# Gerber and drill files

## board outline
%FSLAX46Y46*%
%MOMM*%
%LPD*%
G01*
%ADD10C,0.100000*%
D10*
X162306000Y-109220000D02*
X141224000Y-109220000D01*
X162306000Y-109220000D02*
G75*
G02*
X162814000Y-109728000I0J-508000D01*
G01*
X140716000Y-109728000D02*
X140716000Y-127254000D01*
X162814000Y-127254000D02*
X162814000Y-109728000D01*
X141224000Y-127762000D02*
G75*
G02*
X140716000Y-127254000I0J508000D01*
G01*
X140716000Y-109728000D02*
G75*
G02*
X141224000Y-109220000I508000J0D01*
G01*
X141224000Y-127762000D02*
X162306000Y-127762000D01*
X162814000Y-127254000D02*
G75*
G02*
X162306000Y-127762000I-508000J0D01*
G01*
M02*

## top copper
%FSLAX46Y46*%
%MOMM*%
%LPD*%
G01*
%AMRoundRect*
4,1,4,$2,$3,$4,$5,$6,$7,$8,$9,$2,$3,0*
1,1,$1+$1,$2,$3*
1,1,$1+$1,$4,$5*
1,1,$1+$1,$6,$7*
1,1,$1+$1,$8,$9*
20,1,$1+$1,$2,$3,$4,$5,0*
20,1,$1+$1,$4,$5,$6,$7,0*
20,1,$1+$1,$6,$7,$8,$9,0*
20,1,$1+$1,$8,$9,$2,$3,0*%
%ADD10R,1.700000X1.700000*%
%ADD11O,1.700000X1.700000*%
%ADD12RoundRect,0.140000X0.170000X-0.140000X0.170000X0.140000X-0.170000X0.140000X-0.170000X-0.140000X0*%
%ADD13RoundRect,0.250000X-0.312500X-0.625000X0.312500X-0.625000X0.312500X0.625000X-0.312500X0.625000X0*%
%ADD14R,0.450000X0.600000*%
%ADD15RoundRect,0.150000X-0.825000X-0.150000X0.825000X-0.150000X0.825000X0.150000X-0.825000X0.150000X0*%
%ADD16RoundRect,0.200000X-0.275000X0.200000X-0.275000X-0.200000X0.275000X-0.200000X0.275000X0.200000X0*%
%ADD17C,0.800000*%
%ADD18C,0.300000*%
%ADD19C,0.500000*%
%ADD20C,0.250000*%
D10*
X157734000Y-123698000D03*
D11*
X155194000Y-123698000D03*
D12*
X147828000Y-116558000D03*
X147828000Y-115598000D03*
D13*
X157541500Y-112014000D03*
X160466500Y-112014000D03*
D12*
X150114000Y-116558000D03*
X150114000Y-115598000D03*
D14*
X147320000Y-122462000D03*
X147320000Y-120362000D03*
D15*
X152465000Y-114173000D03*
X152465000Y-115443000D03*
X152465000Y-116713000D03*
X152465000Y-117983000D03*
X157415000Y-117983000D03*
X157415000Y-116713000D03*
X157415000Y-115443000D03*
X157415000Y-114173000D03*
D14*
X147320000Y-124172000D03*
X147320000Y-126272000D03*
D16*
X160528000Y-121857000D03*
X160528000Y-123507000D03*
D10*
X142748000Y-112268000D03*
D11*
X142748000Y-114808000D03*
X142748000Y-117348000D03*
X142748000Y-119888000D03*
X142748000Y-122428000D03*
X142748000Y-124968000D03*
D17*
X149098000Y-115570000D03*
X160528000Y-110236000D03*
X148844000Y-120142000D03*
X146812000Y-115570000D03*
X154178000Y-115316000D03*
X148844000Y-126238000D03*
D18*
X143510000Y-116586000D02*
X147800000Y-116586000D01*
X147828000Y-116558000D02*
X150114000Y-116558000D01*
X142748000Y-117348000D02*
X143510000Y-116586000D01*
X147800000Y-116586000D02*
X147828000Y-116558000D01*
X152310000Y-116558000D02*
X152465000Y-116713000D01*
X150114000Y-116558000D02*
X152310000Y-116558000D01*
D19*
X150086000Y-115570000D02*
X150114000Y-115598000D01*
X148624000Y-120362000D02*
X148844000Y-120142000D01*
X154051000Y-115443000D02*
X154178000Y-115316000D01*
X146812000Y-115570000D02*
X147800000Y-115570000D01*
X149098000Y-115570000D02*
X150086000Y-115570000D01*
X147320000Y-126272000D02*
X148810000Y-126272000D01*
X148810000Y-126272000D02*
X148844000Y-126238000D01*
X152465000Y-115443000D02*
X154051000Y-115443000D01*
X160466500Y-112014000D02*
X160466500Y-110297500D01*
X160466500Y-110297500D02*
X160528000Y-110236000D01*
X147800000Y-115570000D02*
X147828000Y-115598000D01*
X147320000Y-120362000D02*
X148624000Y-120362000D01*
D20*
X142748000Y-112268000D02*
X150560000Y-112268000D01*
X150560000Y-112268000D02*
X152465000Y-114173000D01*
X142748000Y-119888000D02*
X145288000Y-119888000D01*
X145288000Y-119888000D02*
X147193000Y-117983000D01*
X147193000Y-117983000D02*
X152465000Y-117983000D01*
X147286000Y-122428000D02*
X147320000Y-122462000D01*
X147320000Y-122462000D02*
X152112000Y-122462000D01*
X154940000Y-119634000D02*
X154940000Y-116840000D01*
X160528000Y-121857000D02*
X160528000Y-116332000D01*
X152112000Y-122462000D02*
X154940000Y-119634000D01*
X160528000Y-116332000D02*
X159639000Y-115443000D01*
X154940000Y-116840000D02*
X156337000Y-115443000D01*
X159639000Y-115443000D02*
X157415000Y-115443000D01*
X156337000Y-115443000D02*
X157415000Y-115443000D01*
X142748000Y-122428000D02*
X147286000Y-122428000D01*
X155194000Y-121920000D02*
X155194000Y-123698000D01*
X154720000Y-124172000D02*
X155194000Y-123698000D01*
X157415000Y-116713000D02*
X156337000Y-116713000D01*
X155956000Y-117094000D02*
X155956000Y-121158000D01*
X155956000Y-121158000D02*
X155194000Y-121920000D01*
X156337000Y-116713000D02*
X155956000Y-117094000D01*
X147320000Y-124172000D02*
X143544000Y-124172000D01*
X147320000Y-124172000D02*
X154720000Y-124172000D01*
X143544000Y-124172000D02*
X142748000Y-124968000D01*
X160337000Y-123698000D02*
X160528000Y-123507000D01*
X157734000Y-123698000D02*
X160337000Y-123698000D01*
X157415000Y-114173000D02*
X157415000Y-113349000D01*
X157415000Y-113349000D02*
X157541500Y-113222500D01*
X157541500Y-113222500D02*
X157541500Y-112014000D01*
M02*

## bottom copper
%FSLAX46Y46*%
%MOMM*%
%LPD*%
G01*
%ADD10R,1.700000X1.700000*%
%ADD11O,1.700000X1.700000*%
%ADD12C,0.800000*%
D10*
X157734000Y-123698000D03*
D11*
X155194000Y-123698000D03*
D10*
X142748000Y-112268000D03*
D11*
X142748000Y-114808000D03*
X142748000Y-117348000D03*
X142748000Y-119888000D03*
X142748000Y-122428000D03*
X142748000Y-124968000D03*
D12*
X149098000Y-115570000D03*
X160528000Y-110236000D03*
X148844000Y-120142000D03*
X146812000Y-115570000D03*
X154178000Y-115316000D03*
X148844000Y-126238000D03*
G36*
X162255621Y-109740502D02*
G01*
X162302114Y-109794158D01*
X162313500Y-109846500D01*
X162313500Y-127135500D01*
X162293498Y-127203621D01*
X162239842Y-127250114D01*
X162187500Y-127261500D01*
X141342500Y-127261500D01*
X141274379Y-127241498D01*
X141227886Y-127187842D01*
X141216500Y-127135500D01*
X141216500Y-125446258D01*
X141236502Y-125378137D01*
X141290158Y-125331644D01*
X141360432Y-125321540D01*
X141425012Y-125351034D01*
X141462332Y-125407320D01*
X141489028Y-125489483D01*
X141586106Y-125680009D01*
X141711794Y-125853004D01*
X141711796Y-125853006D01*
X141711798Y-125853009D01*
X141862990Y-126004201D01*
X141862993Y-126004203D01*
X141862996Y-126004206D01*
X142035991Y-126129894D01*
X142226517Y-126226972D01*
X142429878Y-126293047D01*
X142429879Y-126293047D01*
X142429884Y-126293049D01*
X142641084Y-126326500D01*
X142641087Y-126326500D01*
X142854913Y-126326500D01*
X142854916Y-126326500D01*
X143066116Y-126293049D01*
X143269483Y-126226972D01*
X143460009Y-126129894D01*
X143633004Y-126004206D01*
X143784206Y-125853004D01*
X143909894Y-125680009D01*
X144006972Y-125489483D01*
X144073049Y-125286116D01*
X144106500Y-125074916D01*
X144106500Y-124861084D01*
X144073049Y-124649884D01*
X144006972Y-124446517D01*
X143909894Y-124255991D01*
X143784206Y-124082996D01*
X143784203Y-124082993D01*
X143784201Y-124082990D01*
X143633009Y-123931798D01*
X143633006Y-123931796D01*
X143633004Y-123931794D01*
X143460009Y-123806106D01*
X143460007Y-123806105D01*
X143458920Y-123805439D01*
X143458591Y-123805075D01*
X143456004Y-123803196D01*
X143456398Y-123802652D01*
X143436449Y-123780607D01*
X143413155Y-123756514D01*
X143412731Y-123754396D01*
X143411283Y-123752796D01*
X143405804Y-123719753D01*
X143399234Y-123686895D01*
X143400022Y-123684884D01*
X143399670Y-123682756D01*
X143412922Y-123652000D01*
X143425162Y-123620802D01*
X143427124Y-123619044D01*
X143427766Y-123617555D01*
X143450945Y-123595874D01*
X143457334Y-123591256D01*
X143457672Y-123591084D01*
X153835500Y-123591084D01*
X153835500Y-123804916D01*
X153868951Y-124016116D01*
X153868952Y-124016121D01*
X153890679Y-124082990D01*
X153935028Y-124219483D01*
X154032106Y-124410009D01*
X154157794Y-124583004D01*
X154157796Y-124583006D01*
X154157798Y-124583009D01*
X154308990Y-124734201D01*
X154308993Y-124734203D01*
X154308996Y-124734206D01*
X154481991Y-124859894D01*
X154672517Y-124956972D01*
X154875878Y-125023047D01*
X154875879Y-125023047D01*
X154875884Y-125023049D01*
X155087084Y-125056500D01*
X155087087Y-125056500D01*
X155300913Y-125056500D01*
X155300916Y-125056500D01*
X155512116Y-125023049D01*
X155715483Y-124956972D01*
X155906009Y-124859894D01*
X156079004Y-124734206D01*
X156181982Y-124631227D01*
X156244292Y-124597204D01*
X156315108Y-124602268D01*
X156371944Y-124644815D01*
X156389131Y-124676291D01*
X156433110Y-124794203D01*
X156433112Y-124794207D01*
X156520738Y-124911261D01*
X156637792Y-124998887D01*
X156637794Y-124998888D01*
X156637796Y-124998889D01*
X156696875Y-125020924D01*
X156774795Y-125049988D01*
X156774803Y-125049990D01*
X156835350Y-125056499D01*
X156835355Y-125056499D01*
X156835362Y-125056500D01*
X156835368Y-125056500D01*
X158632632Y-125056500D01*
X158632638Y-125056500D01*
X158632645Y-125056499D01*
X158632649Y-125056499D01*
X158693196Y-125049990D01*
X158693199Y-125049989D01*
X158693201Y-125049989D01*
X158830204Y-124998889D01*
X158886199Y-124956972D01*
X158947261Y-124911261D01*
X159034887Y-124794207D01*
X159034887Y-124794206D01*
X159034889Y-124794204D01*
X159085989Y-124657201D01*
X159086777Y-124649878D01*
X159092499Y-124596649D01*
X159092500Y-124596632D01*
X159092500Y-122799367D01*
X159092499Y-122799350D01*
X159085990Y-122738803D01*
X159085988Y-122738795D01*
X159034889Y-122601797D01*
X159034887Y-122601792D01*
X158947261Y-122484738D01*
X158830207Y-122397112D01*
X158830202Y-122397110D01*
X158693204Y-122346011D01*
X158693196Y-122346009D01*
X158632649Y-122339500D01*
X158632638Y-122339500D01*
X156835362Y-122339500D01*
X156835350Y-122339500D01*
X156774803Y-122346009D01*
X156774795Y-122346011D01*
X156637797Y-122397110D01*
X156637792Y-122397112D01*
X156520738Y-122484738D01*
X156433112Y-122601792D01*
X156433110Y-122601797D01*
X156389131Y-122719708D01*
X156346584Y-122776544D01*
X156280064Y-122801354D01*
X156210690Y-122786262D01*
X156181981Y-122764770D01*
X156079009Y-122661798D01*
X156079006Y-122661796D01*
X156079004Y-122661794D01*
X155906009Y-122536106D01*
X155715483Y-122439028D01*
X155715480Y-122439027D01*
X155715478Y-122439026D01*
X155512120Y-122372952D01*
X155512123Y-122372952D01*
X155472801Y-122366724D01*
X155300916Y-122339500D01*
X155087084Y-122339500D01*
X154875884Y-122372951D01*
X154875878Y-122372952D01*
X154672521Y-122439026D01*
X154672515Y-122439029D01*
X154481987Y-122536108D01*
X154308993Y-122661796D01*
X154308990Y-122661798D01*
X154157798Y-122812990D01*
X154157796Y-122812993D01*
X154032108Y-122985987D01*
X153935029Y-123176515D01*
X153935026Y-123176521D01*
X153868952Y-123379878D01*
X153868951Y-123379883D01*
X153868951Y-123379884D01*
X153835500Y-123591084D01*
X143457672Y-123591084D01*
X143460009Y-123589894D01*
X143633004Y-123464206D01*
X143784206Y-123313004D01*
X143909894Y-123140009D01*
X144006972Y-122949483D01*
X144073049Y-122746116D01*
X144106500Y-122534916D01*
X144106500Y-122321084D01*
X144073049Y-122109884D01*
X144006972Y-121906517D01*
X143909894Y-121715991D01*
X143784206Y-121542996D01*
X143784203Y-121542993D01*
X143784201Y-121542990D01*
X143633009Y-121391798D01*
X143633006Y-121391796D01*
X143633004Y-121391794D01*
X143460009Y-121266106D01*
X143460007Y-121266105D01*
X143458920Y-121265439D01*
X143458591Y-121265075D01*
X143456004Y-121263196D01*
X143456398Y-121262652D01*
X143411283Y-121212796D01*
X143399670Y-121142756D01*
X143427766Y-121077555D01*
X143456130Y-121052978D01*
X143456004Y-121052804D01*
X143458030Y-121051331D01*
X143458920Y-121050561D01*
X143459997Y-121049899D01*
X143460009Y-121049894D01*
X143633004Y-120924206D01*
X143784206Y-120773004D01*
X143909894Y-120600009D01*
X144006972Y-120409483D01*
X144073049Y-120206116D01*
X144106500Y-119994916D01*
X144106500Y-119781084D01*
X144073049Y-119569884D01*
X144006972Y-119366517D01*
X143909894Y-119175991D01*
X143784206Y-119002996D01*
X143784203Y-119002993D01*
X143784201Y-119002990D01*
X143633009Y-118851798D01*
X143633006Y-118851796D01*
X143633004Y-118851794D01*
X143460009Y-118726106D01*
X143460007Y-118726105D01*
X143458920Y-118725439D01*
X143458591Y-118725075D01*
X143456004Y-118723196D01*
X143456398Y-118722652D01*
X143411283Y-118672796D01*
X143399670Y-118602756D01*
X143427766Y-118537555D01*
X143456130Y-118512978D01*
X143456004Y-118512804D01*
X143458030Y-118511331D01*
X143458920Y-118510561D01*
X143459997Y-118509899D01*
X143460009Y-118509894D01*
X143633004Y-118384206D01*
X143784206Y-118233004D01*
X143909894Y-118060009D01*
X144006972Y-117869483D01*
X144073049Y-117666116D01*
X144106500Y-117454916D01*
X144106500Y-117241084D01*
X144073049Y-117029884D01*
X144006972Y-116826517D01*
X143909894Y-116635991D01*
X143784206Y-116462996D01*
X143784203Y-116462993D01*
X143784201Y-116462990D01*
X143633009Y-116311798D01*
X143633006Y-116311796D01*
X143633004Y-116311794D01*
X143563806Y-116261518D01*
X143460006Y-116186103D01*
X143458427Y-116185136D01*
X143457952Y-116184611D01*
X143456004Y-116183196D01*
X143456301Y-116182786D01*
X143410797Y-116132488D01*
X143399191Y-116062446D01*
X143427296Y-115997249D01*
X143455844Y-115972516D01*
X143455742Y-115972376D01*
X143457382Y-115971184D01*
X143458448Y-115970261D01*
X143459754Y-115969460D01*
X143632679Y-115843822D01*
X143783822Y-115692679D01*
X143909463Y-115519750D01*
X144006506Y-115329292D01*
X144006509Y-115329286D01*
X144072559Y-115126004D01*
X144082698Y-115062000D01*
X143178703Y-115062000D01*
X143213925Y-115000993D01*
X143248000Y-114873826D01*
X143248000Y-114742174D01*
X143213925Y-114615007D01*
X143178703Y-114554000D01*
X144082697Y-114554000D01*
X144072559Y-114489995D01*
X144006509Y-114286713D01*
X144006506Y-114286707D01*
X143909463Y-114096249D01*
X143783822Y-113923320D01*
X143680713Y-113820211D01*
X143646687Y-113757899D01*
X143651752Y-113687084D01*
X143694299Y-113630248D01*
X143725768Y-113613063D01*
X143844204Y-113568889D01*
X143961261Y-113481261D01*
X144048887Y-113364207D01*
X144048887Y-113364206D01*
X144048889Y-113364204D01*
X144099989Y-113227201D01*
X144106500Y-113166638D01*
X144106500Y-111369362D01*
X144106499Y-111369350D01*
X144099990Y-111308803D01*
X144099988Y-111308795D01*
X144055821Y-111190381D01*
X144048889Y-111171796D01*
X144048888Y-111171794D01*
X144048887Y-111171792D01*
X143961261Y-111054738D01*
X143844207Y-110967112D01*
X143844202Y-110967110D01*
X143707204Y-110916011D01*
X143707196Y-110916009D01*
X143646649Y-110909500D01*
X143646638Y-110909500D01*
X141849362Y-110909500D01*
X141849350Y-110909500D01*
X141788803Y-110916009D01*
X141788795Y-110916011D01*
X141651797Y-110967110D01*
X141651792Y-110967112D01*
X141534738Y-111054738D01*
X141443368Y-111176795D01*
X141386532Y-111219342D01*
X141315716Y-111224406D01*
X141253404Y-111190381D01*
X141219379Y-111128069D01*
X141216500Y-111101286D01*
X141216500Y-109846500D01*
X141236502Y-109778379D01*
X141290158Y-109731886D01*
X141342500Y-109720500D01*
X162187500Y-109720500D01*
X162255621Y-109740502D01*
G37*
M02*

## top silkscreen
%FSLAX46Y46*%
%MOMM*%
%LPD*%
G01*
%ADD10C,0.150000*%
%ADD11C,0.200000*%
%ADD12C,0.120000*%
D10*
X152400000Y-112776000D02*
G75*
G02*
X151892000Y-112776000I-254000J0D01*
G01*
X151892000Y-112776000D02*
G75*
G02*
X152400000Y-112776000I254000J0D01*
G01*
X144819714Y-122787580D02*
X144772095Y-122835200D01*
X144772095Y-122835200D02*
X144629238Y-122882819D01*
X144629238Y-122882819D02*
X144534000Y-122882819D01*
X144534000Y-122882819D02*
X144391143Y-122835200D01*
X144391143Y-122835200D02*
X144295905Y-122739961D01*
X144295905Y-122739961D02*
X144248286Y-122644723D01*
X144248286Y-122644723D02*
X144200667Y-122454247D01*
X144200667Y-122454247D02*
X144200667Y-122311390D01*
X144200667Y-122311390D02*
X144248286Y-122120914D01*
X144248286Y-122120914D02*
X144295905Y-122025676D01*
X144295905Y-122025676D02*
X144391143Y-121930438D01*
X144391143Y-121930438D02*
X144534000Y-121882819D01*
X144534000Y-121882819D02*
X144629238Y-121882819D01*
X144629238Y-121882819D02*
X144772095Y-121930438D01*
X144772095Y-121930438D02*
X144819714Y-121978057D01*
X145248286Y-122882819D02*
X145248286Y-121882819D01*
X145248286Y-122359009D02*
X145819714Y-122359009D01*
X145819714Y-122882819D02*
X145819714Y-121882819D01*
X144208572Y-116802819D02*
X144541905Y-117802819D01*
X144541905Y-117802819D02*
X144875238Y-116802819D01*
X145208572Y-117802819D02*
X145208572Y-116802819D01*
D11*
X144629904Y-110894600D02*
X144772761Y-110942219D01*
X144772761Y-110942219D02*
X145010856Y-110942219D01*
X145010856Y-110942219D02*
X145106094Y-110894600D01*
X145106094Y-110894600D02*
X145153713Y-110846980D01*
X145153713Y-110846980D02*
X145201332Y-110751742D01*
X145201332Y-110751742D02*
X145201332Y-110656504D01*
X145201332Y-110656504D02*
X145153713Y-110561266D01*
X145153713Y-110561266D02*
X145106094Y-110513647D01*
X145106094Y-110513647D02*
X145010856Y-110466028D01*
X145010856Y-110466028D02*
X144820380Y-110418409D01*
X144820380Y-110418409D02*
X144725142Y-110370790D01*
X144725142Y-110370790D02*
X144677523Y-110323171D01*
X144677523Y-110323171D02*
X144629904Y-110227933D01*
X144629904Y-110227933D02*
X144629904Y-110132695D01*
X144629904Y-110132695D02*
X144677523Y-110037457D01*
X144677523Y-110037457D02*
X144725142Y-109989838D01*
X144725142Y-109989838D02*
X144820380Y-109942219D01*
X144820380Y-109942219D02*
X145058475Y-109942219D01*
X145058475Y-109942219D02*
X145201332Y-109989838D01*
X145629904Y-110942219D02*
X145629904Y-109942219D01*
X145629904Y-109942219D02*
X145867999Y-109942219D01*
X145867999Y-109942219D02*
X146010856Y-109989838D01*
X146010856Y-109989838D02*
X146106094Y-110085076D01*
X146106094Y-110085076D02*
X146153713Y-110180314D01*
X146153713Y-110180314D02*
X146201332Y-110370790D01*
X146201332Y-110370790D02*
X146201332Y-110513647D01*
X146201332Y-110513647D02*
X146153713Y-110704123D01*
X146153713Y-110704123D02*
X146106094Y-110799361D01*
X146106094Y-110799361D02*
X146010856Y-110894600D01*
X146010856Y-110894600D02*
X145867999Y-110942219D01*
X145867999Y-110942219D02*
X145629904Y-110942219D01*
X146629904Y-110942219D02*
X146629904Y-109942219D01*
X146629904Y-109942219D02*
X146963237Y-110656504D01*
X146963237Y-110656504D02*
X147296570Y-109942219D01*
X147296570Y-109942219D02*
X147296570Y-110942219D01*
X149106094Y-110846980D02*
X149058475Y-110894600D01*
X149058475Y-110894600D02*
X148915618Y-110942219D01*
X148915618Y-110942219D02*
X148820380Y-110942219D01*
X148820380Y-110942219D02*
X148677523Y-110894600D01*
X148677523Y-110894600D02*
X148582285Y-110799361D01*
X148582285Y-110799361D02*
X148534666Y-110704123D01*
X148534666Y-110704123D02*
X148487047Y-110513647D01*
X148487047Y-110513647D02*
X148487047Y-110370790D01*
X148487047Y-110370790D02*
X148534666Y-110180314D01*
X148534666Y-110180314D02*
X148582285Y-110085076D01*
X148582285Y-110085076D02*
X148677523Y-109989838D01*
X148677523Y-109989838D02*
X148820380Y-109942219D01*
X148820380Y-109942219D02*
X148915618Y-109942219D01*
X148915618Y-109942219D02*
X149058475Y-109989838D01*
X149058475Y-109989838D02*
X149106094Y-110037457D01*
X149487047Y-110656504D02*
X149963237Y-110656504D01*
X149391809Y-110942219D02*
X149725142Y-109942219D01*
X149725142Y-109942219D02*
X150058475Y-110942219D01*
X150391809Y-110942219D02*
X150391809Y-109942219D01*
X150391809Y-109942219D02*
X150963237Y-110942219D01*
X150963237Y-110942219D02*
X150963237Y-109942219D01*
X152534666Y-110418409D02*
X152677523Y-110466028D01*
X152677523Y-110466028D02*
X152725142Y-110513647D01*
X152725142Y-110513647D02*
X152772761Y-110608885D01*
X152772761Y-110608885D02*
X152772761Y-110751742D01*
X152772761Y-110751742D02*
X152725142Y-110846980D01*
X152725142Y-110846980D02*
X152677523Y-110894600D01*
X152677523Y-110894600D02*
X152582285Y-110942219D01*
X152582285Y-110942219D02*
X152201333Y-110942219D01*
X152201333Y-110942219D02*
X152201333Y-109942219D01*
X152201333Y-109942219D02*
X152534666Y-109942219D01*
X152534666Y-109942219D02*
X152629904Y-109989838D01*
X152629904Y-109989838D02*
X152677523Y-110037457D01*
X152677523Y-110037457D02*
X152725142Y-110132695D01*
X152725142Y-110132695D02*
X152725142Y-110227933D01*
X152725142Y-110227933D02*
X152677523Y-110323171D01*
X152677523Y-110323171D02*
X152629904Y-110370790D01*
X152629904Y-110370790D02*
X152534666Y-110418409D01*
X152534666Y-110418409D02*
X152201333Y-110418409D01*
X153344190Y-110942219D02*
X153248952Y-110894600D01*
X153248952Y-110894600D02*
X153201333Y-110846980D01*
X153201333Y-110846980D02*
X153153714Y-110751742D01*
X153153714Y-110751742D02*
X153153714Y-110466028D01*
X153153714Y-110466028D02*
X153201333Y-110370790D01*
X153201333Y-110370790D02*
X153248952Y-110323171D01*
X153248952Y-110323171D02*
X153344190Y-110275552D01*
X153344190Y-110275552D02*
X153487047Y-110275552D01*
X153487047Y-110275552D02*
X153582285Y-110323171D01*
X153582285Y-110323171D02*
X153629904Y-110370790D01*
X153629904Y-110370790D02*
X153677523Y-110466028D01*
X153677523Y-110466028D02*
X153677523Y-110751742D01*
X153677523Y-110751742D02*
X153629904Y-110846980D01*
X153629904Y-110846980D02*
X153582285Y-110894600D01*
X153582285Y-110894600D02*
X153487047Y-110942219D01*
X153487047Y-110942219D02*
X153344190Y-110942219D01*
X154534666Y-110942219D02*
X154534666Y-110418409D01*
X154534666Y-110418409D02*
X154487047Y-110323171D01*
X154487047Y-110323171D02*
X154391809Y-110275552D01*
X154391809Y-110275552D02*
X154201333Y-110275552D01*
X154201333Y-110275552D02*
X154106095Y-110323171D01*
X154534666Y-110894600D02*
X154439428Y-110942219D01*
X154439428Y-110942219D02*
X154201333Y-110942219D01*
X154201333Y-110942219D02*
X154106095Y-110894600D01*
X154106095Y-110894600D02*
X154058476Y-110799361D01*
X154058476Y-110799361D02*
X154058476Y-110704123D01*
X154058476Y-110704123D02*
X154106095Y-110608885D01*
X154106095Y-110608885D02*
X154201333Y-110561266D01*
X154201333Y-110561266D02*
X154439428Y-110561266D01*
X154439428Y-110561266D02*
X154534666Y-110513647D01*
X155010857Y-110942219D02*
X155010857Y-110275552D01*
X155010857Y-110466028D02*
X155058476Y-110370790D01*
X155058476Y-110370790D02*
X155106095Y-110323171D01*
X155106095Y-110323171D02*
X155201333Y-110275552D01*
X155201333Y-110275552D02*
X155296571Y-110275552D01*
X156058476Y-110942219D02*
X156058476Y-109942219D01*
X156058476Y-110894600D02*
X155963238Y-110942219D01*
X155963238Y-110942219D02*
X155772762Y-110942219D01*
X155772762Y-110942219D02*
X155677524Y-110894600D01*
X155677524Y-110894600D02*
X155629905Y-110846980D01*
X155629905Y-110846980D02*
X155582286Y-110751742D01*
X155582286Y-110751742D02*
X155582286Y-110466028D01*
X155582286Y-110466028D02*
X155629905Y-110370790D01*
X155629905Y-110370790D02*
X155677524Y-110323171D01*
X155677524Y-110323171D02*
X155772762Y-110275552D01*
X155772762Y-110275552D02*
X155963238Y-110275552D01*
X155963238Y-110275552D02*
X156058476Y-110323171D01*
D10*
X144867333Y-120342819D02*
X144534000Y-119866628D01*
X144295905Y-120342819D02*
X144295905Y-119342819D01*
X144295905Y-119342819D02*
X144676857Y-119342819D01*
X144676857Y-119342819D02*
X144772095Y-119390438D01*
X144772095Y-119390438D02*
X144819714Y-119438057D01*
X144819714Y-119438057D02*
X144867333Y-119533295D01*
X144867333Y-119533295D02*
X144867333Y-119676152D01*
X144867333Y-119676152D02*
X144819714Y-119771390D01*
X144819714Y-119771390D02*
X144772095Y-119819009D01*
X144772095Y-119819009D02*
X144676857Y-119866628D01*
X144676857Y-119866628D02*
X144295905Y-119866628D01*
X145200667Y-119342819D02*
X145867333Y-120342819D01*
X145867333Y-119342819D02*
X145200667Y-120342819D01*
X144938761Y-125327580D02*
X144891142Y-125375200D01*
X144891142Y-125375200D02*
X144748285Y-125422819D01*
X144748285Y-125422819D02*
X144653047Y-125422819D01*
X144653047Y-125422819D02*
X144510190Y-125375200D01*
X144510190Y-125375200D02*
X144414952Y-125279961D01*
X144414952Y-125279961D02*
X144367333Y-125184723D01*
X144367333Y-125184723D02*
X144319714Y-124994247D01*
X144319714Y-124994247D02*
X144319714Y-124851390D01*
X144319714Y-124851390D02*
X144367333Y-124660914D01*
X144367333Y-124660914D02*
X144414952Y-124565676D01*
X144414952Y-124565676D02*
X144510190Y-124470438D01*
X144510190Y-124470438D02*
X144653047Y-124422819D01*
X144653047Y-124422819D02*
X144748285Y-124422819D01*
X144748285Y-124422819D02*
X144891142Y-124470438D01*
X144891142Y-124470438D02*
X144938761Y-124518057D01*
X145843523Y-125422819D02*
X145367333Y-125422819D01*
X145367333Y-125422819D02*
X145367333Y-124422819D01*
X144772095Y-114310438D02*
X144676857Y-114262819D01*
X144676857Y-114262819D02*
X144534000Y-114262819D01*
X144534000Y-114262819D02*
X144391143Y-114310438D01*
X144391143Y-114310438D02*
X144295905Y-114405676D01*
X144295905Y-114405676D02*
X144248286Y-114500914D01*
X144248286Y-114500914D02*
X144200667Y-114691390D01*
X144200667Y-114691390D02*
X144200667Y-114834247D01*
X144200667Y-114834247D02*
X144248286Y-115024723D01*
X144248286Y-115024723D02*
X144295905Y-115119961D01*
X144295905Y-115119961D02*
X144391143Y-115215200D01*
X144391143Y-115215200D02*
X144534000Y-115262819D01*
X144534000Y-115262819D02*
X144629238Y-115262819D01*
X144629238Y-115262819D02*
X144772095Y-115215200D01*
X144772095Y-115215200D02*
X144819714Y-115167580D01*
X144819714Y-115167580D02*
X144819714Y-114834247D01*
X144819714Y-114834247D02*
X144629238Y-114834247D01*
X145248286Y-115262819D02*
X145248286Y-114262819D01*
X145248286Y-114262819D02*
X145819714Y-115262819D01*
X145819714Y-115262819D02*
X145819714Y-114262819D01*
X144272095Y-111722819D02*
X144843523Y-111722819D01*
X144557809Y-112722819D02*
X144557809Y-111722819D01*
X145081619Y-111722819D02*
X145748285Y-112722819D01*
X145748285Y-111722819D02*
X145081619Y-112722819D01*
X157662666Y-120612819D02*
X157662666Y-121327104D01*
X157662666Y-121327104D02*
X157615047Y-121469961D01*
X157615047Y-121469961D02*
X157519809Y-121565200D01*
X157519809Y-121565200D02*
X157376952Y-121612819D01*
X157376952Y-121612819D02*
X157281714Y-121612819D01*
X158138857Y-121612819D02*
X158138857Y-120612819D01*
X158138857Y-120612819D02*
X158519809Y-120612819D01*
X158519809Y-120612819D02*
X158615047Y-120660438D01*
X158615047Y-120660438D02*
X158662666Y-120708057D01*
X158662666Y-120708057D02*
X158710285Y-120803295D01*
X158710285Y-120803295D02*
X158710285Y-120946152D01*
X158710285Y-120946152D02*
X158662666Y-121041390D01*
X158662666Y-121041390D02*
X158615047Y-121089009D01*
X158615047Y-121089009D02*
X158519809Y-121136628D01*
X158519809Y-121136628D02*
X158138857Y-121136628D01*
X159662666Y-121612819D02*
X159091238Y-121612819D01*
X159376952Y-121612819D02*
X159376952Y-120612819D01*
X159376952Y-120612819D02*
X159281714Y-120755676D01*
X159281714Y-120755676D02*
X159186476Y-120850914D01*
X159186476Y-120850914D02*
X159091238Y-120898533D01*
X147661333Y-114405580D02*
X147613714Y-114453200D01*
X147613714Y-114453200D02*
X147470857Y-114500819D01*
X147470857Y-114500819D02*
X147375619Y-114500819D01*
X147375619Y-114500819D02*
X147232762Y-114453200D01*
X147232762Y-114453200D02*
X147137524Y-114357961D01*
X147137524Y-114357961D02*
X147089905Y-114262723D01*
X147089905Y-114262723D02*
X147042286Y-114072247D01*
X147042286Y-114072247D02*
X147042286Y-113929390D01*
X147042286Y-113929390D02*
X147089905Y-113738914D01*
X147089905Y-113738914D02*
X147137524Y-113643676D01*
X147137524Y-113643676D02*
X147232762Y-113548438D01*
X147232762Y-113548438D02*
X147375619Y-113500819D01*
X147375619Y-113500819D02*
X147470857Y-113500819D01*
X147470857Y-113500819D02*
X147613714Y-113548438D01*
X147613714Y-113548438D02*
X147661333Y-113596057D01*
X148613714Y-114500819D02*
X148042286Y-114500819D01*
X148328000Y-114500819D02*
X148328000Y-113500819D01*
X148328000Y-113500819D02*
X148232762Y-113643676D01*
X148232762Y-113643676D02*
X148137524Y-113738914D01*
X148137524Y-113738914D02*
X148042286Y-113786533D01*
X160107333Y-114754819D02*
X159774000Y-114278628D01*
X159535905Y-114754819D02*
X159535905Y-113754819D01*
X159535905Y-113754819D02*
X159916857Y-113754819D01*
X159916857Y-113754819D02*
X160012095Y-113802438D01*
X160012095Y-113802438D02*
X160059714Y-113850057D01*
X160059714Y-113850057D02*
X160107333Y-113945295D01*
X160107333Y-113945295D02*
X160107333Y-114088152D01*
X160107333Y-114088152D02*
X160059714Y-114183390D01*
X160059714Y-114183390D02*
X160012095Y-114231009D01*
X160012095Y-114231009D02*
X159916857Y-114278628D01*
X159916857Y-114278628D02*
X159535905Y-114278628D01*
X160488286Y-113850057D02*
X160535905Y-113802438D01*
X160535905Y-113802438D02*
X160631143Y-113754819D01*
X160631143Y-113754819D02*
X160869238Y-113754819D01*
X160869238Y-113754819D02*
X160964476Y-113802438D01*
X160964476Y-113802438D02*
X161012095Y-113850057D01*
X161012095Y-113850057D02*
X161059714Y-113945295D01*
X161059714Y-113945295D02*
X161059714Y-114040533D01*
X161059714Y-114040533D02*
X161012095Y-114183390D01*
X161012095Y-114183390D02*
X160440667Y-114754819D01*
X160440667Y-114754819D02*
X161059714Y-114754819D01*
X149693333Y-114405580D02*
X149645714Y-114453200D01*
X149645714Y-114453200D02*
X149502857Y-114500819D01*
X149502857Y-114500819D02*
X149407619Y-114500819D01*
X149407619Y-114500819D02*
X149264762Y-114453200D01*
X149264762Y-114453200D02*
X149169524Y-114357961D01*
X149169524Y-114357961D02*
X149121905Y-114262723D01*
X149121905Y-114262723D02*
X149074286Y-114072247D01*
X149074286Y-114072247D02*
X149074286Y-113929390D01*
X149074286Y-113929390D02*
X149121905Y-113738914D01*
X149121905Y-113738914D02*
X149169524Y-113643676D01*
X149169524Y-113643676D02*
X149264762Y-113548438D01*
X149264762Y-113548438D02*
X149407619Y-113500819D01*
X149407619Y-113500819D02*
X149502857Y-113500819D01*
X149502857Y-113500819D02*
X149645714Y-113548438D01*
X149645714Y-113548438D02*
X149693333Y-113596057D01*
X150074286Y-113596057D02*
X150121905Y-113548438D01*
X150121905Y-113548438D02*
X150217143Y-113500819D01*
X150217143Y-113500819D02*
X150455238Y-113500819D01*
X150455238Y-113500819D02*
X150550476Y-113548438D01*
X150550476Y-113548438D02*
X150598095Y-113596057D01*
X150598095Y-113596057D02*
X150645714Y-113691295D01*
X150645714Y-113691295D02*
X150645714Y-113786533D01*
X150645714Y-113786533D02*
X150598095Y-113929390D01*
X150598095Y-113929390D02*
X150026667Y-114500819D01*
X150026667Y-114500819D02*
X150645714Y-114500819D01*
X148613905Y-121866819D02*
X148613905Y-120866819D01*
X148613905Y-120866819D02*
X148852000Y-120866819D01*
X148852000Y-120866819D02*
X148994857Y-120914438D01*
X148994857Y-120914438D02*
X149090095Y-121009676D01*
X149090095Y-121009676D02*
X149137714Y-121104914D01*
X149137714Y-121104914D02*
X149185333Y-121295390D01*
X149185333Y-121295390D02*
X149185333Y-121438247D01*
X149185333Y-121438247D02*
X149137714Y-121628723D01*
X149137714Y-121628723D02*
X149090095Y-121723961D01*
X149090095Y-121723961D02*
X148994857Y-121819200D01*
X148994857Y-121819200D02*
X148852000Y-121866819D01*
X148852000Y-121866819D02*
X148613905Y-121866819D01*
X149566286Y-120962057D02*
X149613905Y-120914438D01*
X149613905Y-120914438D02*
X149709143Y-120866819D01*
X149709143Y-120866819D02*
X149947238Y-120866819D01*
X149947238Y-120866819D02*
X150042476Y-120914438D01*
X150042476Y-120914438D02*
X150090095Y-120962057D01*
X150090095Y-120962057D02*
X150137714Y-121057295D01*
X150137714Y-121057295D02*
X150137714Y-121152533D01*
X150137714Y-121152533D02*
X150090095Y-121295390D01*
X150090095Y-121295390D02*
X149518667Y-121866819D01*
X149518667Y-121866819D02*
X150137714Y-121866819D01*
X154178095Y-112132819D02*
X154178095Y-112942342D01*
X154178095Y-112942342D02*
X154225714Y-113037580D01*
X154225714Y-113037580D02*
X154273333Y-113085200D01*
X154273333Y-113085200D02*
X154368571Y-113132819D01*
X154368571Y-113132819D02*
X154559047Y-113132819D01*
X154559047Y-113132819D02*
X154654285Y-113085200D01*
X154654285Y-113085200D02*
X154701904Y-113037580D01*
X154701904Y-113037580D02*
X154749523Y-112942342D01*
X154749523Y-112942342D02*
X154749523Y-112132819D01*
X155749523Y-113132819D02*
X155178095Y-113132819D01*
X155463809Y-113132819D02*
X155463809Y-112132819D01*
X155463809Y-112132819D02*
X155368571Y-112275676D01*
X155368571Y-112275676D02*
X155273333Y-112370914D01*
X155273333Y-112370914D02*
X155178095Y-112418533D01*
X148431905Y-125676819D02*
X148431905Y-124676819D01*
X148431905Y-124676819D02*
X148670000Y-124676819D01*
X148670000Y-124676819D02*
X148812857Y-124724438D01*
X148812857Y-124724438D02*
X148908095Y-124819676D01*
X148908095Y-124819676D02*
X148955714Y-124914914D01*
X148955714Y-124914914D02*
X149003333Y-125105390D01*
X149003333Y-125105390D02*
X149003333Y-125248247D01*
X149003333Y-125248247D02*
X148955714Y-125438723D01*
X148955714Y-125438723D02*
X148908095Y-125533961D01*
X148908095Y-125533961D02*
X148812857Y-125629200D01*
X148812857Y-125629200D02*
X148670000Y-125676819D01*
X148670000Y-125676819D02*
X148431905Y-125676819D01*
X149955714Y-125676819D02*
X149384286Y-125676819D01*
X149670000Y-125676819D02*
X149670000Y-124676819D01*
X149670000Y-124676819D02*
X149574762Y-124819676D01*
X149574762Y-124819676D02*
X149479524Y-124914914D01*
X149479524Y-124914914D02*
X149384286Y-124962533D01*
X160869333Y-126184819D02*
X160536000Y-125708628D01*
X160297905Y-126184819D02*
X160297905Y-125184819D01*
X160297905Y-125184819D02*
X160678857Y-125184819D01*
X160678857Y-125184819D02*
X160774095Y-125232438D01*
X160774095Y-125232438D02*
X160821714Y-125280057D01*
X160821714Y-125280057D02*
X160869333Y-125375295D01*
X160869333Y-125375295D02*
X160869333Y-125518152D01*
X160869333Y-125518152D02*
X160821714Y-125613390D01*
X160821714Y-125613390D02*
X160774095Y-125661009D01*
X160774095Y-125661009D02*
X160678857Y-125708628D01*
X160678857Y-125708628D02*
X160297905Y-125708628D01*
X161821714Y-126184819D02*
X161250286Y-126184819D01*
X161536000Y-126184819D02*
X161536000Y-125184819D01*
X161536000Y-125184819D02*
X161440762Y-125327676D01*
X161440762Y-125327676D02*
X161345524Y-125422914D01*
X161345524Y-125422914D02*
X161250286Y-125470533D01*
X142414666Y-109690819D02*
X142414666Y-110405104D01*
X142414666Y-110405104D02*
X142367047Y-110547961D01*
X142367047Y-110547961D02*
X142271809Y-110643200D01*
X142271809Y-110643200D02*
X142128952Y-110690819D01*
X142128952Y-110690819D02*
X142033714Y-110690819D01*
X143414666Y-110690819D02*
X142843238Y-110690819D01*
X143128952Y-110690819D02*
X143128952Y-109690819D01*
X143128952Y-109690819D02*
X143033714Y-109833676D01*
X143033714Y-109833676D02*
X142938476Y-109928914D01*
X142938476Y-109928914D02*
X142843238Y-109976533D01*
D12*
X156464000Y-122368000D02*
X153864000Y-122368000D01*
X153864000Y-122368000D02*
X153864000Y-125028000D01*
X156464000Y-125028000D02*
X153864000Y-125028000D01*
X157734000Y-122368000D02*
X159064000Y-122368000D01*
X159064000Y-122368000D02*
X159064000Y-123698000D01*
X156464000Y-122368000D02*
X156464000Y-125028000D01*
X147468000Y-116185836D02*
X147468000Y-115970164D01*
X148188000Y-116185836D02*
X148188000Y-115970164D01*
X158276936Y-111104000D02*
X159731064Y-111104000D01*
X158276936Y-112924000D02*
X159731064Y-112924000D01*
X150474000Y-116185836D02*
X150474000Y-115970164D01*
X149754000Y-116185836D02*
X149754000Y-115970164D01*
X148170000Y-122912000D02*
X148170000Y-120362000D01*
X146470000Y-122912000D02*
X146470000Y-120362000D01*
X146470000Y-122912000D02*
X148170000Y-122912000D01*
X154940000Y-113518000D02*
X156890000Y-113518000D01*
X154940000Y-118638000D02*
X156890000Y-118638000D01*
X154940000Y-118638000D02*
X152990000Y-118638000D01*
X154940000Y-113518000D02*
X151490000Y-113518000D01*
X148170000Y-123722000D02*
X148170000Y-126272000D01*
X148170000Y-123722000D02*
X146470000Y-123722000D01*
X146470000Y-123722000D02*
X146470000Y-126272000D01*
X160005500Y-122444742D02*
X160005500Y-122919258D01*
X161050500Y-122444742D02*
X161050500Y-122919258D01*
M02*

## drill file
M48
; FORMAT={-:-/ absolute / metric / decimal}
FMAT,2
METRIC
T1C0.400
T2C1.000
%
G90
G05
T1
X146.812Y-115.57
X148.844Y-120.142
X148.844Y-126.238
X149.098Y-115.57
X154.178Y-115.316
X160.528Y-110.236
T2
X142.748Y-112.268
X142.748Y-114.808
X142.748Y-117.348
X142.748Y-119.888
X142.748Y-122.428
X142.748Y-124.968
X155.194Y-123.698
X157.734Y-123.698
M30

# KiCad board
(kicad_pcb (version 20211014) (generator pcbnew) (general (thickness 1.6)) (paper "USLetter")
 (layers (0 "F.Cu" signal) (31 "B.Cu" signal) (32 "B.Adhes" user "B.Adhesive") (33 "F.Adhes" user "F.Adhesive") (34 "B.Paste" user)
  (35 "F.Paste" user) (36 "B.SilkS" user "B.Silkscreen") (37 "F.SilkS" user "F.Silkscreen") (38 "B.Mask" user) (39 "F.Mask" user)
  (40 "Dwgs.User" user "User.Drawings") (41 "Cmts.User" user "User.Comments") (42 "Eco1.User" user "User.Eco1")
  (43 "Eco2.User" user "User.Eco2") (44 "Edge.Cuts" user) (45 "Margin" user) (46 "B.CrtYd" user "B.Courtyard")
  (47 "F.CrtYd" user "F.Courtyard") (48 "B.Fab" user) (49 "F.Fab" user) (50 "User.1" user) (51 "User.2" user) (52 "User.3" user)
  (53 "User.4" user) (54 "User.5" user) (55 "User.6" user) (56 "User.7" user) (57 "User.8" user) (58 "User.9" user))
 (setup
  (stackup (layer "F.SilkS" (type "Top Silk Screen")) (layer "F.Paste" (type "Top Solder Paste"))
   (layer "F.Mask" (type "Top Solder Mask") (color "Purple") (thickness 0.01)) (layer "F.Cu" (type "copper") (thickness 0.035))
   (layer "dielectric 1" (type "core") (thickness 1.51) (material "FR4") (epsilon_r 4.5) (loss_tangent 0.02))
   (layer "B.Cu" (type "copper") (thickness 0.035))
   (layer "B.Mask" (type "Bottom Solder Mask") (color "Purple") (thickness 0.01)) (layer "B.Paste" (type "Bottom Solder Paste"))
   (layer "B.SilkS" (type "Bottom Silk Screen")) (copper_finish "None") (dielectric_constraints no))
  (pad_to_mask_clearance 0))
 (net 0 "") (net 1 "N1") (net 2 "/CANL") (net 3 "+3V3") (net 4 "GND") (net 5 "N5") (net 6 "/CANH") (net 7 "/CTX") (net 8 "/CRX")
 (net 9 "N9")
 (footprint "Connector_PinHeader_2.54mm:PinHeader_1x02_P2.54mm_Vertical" (layer "F.Cu") (at 157.734 123.698 -90)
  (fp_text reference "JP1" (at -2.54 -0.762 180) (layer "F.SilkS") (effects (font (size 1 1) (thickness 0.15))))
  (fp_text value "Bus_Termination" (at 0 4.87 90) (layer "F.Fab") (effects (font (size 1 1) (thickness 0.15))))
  (fp_line (start -1.33 1.27) (end -1.33 3.87) (layer "F.SilkS") (width 0.12))
  (fp_line (start -1.33 3.87) (end 1.33 3.87) (layer "F.SilkS") (width 0.12))
  (fp_line (start 1.33 1.27) (end 1.33 3.87) (layer "F.SilkS") (width 0.12))
  (fp_line (start -1.33 0) (end -1.33 -1.33) (layer "F.SilkS") (width 0.12))
  (fp_line (start -1.33 -1.33) (end 0 -1.33) (layer "F.SilkS") (width 0.12))
  (fp_line (start -1.33 1.27) (end 1.33 1.27) (layer "F.SilkS") (width 0.12))
  (pad "1" thru_hole rect (at 0 0 270) (size 1.7 1.7) (drill 1) (layers *.Cu *.Mask) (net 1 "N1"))
  (pad "2" thru_hole oval (at 0 2.54 270) (size 1.7 1.7) (drill 1) (layers *.Cu *.Mask) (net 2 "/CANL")))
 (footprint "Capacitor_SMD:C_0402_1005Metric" (layer "F.Cu") (at 147.828 116.078 90)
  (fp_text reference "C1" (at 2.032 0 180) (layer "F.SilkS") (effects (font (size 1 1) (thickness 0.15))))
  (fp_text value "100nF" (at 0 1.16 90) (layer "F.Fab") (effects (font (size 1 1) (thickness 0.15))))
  (fp_line (start -0.107836 -0.36) (end 0.107836 -0.36) (layer "F.SilkS") (width 0.12))
  (fp_line (start -0.107836 0.36) (end 0.107836 0.36) (layer "F.SilkS") (width 0.12))
  (pad "1" smd roundrect (at -0.48 0 90) (size 0.56 0.62) (layers "F.Cu" "F.Paste" "F.Mask") (roundrect_rratio 0.25) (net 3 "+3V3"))
  (pad "2" smd roundrect (at 0.48 0 90) (size 0.56 0.62) (layers "F.Cu" "F.Paste" "F.Mask") (roundrect_rratio 0.25) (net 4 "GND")))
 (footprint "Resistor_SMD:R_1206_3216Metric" (layer "F.Cu") (at 159.004 112.014)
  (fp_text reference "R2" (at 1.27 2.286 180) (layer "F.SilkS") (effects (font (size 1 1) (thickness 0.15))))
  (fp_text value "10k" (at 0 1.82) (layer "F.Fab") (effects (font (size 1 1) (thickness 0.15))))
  (fp_line (start -0.727064 -0.91) (end 0.727064 -0.91) (layer "F.SilkS") (width 0.12))
  (fp_line (start -0.727064 0.91) (end 0.727064 0.91) (layer "F.SilkS") (width 0.12))
  (pad "1" smd roundrect (at -1.4625 0) (size 1.125 1.75) (layers "F.Cu" "F.Paste" "F.Mask") (roundrect_rratio 0.2222222222) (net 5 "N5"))
  (pad "2" smd roundrect (at 1.4625 0) (size 1.125 1.75) (layers "F.Cu" "F.Paste" "F.Mask") (roundrect_rratio 0.2222222222) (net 4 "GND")))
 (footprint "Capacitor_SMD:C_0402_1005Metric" (layer "F.Cu") (at 150.114 116.078 90)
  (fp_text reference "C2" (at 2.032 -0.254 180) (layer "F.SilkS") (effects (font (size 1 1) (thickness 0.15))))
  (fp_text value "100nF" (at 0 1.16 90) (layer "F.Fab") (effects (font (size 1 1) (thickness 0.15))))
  (fp_line (start -0.107836 0.36) (end 0.107836 0.36) (layer "F.SilkS") (width 0.12))
  (fp_line (start -0.107836 -0.36) (end 0.107836 -0.36) (layer "F.SilkS") (width 0.12))
  (pad "1" smd roundrect (at -0.48 0 90) (size 0.56 0.62) (layers "F.Cu" "F.Paste" "F.Mask") (roundrect_rratio 0.25) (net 3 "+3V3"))
  (pad "2" smd roundrect (at 0.48 0 90) (size 0.56 0.62) (layers "F.Cu" "F.Paste" "F.Mask") (roundrect_rratio 0.25) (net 4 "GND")))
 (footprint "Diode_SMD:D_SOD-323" (layer "F.Cu") (at 147.32 121.412 90)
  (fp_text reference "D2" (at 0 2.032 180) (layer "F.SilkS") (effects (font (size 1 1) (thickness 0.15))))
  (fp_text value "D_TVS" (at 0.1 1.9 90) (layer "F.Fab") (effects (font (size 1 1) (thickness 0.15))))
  (fp_line (start -1.5 0.85) (end 1.05 0.85) (layer "F.SilkS") (width 0.12))
  (fp_line (start -1.5 -0.85) (end 1.05 -0.85) (layer "F.SilkS") (width 0.12))
  (fp_line (start -1.5 -0.85) (end -1.5 0.85) (layer "F.SilkS") (width 0.12))
  (pad "1" smd rect (at -1.05 0 90) (size 0.6 0.45) (layers "F.Cu" "F.Paste" "F.Mask") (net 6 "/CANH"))
  (pad "2" smd rect (at 1.05 0 90) (size 0.6 0.45) (layers "F.Cu" "F.Paste" "F.Mask") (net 4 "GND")))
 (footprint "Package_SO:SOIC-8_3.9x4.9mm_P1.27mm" (layer "F.Cu") (at 154.94 116.078)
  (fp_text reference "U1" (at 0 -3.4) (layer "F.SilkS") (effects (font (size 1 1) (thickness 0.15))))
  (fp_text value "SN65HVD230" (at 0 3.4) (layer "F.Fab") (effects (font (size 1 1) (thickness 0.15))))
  (fp_line (start 0 -2.56) (end 1.95 -2.56) (layer "F.SilkS") (width 0.12))
  (fp_line (start 0 2.56) (end 1.95 2.56) (layer "F.SilkS") (width 0.12))
  (fp_line (start 0 2.56) (end -1.95 2.56) (layer "F.SilkS") (width 0.12))
  (fp_line (start 0 -2.56) (end -3.45 -2.56) (layer "F.SilkS") (width 0.12))
  (pad "1" smd roundrect (at -2.475 -1.905) (size 1.95 0.6) (layers "F.Cu" "F.Paste" "F.Mask") (roundrect_rratio 0.25) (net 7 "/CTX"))
  (pad "2" smd roundrect (at -2.475 -0.635) (size 1.95 0.6) (layers "F.Cu" "F.Paste" "F.Mask") (roundrect_rratio 0.25) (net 4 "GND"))
  (pad "3" smd roundrect (at -2.475 0.635) (size 1.95 0.6) (layers "F.Cu" "F.Paste" "F.Mask") (roundrect_rratio 0.25) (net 3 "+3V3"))
  (pad "4" smd roundrect (at -2.475 1.905) (size 1.95 0.6) (layers "F.Cu" "F.Paste" "F.Mask") (roundrect_rratio 0.25) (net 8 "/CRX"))
  (pad "5" smd roundrect (at 2.475 1.905) (size 1.95 0.6) (layers "F.Cu" "F.Paste" "F.Mask") (roundrect_rratio 0.25) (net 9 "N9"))
  (pad "6" smd roundrect (at 2.475 0.635) (size 1.95 0.6) (layers "F.Cu" "F.Paste" "F.Mask") (roundrect_rratio 0.25) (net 2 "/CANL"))
  (pad "7" smd roundrect (at 2.475 -0.635) (size 1.95 0.6) (layers "F.Cu" "F.Paste" "F.Mask") (roundrect_rratio 0.25) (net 6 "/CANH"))
  (pad "8" smd roundrect (at 2.475 -1.905) (size 1.95 0.6) (layers "F.Cu" "F.Paste" "F.Mask") (roundrect_rratio 0.25) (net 5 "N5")))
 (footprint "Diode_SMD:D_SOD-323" (layer "F.Cu") (at 147.32 125.222 -90)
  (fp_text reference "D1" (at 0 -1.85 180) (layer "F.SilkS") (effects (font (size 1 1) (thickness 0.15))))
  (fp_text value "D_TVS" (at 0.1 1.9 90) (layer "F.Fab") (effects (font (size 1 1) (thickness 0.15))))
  (fp_line (start -1.5 -0.85) (end 1.05 -0.85) (layer "F.SilkS") (width 0.12))
  (fp_line (start -1.5 -0.85) (end -1.5 0.85) (layer "F.SilkS") (width 0.12))
  (fp_line (start -1.5 0.85) (end 1.05 0.85) (layer "F.SilkS") (width 0.12))
  (pad "1" smd rect (at -1.05 0 270) (size 0.6 0.45) (layers "F.Cu" "F.Paste" "F.Mask") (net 2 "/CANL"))
  (pad "2" smd rect (at 1.05 0 270) (size 0.6 0.45) (layers "F.Cu" "F.Paste" "F.Mask") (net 4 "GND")))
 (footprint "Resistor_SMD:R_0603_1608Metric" (layer "F.Cu") (at 160.528 122.682 -90)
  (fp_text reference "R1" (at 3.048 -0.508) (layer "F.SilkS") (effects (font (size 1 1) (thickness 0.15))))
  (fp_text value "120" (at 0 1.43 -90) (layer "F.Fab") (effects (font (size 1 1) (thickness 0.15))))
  (fp_line (start -0.237258 0.5225) (end 0.237258 0.5225) (layer "F.SilkS") (width 0.12))
  (fp_line (start -0.237258 -0.5225) (end 0.237258 -0.5225) (layer "F.SilkS") (width 0.12))
  (pad "1" smd roundrect (at -0.825 0 270) (size 0.8 0.95) (layers "F.Cu" "F.Paste" "F.Mask") (roundrect_rratio 0.25) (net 6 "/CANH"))
  (pad "2" smd roundrect (at 0.825 0 270) (size 0.8 0.95) (layers "F.Cu" "F.Paste" "F.Mask") (roundrect_rratio 0.25) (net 1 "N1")))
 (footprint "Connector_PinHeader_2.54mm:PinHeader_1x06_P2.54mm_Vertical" (layer "B.Cu") (at 142.748 112.268 180)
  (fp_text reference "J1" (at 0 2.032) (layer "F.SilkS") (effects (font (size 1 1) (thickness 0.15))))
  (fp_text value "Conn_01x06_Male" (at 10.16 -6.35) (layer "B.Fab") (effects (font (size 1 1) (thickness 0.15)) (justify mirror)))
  (pad "1" thru_hole rect (at 0 0 180) (size 1.7 1.7) (drill 1) (layers *.Cu *.Mask) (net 7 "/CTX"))
  (pad "2" thru_hole oval (at 0 -2.54 180) (size 1.7 1.7) (drill 1) (layers *.Cu *.Mask) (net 4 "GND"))
  (pad "3" thru_hole oval (at 0 -5.08 180) (size 1.7 1.7) (drill 1) (layers *.Cu *.Mask) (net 3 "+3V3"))
  (pad "4" thru_hole oval (at 0 -7.62 180) (size 1.7 1.7) (drill 1) (layers *.Cu *.Mask) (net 8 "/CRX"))
  (pad "5" thru_hole oval (at 0 -10.16 180) (size 1.7 1.7) (drill 1) (layers *.Cu *.Mask) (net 6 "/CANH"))
  (pad "6" thru_hole oval (at 0 -12.7 180) (size 1.7 1.7) (drill 1) (layers *.Cu *.Mask) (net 2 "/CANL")))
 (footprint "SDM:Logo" (layer "B.Cu") (at 156.718 118.364 180)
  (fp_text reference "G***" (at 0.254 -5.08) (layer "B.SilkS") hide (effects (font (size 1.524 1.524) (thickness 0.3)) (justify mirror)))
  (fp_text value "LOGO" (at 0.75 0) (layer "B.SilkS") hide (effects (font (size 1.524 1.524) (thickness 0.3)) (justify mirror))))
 (gr_circle (center 152.146 112.776) (end 152.146 112.522) (layer "F.SilkS") (width 0.15) (fill none))
 (gr_line (start 162.306 109.22) (end 141.224 109.22) (layer "Edge.Cuts") (width 0.1))
 (gr_arc (start 162.306 109.22) (mid 162.66521 109.36879) (end 162.814 109.728) (layer "Edge.Cuts") (width 0.1))
 (gr_line (start 140.716 109.728) (end 140.716 127.254) (layer "Edge.Cuts") (width 0.1))
 (gr_line (start 162.814 127.254) (end 162.814 109.728) (layer "Edge.Cuts") (width 0.1))
 (gr_arc (start 141.224 127.762) (mid 140.86479 127.61321) (end 140.716 127.254) (layer "Edge.Cuts") (width 0.1))
 (gr_arc (start 140.716 109.728) (mid 140.86479 109.36879) (end 141.224 109.22) (layer "Edge.Cuts") (width 0.1))
 (gr_line (start 141.224 127.762) (end 162.306 127.762) (layer "Edge.Cuts") (width 0.1))
 (gr_arc (start 162.814 127.254) (mid 162.66521 127.61321) (end 162.306 127.762) (layer "Edge.Cuts") (width 0.1))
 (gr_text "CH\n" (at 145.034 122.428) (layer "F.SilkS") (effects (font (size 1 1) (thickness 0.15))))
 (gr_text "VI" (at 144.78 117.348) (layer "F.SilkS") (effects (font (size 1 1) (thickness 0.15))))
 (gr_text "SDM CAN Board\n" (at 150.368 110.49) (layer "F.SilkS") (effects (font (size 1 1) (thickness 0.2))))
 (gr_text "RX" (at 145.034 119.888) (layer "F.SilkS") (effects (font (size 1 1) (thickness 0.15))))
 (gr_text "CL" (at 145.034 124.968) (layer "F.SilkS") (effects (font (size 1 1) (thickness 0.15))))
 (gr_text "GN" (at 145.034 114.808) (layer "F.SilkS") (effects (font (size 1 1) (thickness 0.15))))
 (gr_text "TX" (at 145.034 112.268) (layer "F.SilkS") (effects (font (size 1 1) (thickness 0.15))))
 (segment (start 143.51 116.586) (end 147.8 116.586) (width 0.3) (layer "F.Cu") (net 3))
 (segment (start 147.828 116.558) (end 150.114 116.558) (width 0.3) (layer "F.Cu") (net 3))
 (segment (start 142.748 117.348) (end 143.51 116.586) (width 0.3) (layer "F.Cu") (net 3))
 (segment (start 147.8 116.586) (end 147.828 116.558) (width 0.3) (layer "F.Cu") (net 3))
 (segment (start 152.31 116.558) (end 152.465 116.713) (width 0.3) (layer "F.Cu") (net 3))
 (segment (start 150.114 116.558) (end 152.31 116.558) (width 0.3) (layer "F.Cu") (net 3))
 (segment (start 150.086 115.57) (end 150.114 115.598) (width 0.5) (layer "F.Cu") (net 4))
 (segment (start 148.624 120.362) (end 148.844 120.142) (width 0.5) (layer "F.Cu") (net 4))
 (segment (start 154.051 115.443) (end 154.178 115.316) (width 0.5) (layer "F.Cu") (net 4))
 (segment (start 146.812 115.57) (end 147.8 115.57) (width 0.5) (layer "F.Cu") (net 4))
 (segment (start 149.098 115.57) (end 150.086 115.57) (width 0.5) (layer "F.Cu") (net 4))
 (segment (start 147.32 126.272) (end 148.81 126.272) (width 0.5) (layer "F.Cu") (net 4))
 (segment (start 148.81 126.272) (end 148.844 126.238) (width 0.5) (layer "F.Cu") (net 4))
 (segment (start 152.465 115.443) (end 154.051 115.443) (width 0.5) (layer "F.Cu") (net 4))
 (segment (start 160.4665 112.014) (end 160.4665 110.2975) (width 0.5) (layer "F.Cu") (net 4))
 (segment (start 160.4665 110.2975) (end 160.528 110.236) (width 0.5) (layer "F.Cu") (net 4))
 (segment (start 147.8 115.57) (end 147.828 115.598) (width 0.5) (layer "F.Cu") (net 4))
 (segment (start 147.32 120.362) (end 148.624 120.362) (width 0.5) (layer "F.Cu") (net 4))
 (via (at 149.098 115.57) (size 0.8) (drill 0.4) (layers "F.Cu" "B.Cu") (free) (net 4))
 (via (at 160.528 110.236) (size 0.8) (drill 0.4) (layers "F.Cu" "B.Cu") (free) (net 4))
 (via (at 148.844 120.142) (size 0.8) (drill 0.4) (layers "F.Cu" "B.Cu") (free) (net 4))
 (via (at 146.812 115.57) (size 0.8) (drill 0.4) (layers "F.Cu" "B.Cu") (free) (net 4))
 (via (at 154.178 115.316) (size 0.8) (drill 0.4) (layers "F.Cu" "B.Cu") (free) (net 4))
 (via (at 148.844 126.238) (size 0.8) (drill 0.4) (layers "F.Cu" "B.Cu") (free) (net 4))
 (segment (start 142.748 112.268) (end 150.56 112.268) (width 0.25) (layer "F.Cu") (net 7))
 (segment (start 150.56 112.268) (end 152.465 114.173) (width 0.25) (layer "F.Cu") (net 7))
 (segment (start 142.748 119.888) (end 145.288 119.888) (width 0.25) (layer "F.Cu") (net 8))
 (segment (start 145.288 119.888) (end 147.193 117.983) (width 0.25) (layer "F.Cu") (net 8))
 (segment (start 147.193 117.983) (end 152.465 117.983) (width 0.25) (layer "F.Cu") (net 8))
 (segment (start 147.286 122.428) (end 147.32 122.462) (width 0.25) (layer "F.Cu") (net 6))
 (segment (start 147.32 122.462) (end 152.112 122.462) (width 0.25) (layer "F.Cu") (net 6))
 (segment (start 154.94 119.634) (end 154.94 116.84) (width 0.25) (layer "F.Cu") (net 6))
 (segment (start 160.528 121.857) (end 160.528 116.332) (width 0.25) (layer "F.Cu") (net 6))
 (segment (start 152.112 122.462) (end 154.94 119.634) (width 0.25) (layer "F.Cu") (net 6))
 (segment (start 160.528 116.332) (end 159.639 115.443) (width 0.25) (layer "F.Cu") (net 6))
 (segment (start 154.94 116.84) (end 156.337 115.443) (width 0.25) (layer "F.Cu") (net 6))
 (segment (start 159.639 115.443) (end 157.415 115.443) (width 0.25) (layer "F.Cu") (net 6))
 (segment (start 156.337 115.443) (end 157.415 115.443) (width 0.25) (layer "F.Cu") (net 6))
 (segment (start 142.748 122.428) (end 147.286 122.428) (width 0.25) (layer "F.Cu") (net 6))
 (segment (start 155.194 121.92) (end 155.194 123.698) (width 0.25) (layer "F.Cu") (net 2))
 (segment (start 154.72 124.172) (end 155.194 123.698) (width 0.25) (layer "F.Cu") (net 2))
 (segment (start 157.415 116.713) (end 156.337 116.713) (width 0.25) (layer "F.Cu") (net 2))
 (segment (start 155.956 117.094) (end 155.956 121.158) (width 0.25) (layer "F.Cu") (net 2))
 (segment (start 155.956 121.158) (end 155.194 121.92) (width 0.25) (layer "F.Cu") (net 2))
 (segment (start 156.337 116.713) (end 155.956 117.094) (width 0.25) (layer "F.Cu") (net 2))
 (segment (start 147.32 124.172) (end 143.544 124.172) (width 0.25) (layer "F.Cu") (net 2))
 (segment (start 147.32 124.172) (end 154.72 124.172) (width 0.25) (layer "F.Cu") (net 2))
 (segment (start 143.544 124.172) (end 142.748 124.968) (width 0.25) (layer "F.Cu") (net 2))
 (segment (start 160.337 123.698) (end 160.528 123.507) (width 0.25) (layer "F.Cu") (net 1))
 (segment (start 157.734 123.698) (end 160.337 123.698) (width 0.25) (layer "F.Cu") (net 1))
 (segment (start 157.415 114.173) (end 157.415 113.349) (width 0.25) (layer "F.Cu") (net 5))
 (segment (start 157.415 113.349) (end 157.5415 113.2225) (width 0.25) (layer "F.Cu") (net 5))
 (segment (start 157.5415 113.2225) (end 157.5415 112.014) (width 0.25) (layer "F.Cu") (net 5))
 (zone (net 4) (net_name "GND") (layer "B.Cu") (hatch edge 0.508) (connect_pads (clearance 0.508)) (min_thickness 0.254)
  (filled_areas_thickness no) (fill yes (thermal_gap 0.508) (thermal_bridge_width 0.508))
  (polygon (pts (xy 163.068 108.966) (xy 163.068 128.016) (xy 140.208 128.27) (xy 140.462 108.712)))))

